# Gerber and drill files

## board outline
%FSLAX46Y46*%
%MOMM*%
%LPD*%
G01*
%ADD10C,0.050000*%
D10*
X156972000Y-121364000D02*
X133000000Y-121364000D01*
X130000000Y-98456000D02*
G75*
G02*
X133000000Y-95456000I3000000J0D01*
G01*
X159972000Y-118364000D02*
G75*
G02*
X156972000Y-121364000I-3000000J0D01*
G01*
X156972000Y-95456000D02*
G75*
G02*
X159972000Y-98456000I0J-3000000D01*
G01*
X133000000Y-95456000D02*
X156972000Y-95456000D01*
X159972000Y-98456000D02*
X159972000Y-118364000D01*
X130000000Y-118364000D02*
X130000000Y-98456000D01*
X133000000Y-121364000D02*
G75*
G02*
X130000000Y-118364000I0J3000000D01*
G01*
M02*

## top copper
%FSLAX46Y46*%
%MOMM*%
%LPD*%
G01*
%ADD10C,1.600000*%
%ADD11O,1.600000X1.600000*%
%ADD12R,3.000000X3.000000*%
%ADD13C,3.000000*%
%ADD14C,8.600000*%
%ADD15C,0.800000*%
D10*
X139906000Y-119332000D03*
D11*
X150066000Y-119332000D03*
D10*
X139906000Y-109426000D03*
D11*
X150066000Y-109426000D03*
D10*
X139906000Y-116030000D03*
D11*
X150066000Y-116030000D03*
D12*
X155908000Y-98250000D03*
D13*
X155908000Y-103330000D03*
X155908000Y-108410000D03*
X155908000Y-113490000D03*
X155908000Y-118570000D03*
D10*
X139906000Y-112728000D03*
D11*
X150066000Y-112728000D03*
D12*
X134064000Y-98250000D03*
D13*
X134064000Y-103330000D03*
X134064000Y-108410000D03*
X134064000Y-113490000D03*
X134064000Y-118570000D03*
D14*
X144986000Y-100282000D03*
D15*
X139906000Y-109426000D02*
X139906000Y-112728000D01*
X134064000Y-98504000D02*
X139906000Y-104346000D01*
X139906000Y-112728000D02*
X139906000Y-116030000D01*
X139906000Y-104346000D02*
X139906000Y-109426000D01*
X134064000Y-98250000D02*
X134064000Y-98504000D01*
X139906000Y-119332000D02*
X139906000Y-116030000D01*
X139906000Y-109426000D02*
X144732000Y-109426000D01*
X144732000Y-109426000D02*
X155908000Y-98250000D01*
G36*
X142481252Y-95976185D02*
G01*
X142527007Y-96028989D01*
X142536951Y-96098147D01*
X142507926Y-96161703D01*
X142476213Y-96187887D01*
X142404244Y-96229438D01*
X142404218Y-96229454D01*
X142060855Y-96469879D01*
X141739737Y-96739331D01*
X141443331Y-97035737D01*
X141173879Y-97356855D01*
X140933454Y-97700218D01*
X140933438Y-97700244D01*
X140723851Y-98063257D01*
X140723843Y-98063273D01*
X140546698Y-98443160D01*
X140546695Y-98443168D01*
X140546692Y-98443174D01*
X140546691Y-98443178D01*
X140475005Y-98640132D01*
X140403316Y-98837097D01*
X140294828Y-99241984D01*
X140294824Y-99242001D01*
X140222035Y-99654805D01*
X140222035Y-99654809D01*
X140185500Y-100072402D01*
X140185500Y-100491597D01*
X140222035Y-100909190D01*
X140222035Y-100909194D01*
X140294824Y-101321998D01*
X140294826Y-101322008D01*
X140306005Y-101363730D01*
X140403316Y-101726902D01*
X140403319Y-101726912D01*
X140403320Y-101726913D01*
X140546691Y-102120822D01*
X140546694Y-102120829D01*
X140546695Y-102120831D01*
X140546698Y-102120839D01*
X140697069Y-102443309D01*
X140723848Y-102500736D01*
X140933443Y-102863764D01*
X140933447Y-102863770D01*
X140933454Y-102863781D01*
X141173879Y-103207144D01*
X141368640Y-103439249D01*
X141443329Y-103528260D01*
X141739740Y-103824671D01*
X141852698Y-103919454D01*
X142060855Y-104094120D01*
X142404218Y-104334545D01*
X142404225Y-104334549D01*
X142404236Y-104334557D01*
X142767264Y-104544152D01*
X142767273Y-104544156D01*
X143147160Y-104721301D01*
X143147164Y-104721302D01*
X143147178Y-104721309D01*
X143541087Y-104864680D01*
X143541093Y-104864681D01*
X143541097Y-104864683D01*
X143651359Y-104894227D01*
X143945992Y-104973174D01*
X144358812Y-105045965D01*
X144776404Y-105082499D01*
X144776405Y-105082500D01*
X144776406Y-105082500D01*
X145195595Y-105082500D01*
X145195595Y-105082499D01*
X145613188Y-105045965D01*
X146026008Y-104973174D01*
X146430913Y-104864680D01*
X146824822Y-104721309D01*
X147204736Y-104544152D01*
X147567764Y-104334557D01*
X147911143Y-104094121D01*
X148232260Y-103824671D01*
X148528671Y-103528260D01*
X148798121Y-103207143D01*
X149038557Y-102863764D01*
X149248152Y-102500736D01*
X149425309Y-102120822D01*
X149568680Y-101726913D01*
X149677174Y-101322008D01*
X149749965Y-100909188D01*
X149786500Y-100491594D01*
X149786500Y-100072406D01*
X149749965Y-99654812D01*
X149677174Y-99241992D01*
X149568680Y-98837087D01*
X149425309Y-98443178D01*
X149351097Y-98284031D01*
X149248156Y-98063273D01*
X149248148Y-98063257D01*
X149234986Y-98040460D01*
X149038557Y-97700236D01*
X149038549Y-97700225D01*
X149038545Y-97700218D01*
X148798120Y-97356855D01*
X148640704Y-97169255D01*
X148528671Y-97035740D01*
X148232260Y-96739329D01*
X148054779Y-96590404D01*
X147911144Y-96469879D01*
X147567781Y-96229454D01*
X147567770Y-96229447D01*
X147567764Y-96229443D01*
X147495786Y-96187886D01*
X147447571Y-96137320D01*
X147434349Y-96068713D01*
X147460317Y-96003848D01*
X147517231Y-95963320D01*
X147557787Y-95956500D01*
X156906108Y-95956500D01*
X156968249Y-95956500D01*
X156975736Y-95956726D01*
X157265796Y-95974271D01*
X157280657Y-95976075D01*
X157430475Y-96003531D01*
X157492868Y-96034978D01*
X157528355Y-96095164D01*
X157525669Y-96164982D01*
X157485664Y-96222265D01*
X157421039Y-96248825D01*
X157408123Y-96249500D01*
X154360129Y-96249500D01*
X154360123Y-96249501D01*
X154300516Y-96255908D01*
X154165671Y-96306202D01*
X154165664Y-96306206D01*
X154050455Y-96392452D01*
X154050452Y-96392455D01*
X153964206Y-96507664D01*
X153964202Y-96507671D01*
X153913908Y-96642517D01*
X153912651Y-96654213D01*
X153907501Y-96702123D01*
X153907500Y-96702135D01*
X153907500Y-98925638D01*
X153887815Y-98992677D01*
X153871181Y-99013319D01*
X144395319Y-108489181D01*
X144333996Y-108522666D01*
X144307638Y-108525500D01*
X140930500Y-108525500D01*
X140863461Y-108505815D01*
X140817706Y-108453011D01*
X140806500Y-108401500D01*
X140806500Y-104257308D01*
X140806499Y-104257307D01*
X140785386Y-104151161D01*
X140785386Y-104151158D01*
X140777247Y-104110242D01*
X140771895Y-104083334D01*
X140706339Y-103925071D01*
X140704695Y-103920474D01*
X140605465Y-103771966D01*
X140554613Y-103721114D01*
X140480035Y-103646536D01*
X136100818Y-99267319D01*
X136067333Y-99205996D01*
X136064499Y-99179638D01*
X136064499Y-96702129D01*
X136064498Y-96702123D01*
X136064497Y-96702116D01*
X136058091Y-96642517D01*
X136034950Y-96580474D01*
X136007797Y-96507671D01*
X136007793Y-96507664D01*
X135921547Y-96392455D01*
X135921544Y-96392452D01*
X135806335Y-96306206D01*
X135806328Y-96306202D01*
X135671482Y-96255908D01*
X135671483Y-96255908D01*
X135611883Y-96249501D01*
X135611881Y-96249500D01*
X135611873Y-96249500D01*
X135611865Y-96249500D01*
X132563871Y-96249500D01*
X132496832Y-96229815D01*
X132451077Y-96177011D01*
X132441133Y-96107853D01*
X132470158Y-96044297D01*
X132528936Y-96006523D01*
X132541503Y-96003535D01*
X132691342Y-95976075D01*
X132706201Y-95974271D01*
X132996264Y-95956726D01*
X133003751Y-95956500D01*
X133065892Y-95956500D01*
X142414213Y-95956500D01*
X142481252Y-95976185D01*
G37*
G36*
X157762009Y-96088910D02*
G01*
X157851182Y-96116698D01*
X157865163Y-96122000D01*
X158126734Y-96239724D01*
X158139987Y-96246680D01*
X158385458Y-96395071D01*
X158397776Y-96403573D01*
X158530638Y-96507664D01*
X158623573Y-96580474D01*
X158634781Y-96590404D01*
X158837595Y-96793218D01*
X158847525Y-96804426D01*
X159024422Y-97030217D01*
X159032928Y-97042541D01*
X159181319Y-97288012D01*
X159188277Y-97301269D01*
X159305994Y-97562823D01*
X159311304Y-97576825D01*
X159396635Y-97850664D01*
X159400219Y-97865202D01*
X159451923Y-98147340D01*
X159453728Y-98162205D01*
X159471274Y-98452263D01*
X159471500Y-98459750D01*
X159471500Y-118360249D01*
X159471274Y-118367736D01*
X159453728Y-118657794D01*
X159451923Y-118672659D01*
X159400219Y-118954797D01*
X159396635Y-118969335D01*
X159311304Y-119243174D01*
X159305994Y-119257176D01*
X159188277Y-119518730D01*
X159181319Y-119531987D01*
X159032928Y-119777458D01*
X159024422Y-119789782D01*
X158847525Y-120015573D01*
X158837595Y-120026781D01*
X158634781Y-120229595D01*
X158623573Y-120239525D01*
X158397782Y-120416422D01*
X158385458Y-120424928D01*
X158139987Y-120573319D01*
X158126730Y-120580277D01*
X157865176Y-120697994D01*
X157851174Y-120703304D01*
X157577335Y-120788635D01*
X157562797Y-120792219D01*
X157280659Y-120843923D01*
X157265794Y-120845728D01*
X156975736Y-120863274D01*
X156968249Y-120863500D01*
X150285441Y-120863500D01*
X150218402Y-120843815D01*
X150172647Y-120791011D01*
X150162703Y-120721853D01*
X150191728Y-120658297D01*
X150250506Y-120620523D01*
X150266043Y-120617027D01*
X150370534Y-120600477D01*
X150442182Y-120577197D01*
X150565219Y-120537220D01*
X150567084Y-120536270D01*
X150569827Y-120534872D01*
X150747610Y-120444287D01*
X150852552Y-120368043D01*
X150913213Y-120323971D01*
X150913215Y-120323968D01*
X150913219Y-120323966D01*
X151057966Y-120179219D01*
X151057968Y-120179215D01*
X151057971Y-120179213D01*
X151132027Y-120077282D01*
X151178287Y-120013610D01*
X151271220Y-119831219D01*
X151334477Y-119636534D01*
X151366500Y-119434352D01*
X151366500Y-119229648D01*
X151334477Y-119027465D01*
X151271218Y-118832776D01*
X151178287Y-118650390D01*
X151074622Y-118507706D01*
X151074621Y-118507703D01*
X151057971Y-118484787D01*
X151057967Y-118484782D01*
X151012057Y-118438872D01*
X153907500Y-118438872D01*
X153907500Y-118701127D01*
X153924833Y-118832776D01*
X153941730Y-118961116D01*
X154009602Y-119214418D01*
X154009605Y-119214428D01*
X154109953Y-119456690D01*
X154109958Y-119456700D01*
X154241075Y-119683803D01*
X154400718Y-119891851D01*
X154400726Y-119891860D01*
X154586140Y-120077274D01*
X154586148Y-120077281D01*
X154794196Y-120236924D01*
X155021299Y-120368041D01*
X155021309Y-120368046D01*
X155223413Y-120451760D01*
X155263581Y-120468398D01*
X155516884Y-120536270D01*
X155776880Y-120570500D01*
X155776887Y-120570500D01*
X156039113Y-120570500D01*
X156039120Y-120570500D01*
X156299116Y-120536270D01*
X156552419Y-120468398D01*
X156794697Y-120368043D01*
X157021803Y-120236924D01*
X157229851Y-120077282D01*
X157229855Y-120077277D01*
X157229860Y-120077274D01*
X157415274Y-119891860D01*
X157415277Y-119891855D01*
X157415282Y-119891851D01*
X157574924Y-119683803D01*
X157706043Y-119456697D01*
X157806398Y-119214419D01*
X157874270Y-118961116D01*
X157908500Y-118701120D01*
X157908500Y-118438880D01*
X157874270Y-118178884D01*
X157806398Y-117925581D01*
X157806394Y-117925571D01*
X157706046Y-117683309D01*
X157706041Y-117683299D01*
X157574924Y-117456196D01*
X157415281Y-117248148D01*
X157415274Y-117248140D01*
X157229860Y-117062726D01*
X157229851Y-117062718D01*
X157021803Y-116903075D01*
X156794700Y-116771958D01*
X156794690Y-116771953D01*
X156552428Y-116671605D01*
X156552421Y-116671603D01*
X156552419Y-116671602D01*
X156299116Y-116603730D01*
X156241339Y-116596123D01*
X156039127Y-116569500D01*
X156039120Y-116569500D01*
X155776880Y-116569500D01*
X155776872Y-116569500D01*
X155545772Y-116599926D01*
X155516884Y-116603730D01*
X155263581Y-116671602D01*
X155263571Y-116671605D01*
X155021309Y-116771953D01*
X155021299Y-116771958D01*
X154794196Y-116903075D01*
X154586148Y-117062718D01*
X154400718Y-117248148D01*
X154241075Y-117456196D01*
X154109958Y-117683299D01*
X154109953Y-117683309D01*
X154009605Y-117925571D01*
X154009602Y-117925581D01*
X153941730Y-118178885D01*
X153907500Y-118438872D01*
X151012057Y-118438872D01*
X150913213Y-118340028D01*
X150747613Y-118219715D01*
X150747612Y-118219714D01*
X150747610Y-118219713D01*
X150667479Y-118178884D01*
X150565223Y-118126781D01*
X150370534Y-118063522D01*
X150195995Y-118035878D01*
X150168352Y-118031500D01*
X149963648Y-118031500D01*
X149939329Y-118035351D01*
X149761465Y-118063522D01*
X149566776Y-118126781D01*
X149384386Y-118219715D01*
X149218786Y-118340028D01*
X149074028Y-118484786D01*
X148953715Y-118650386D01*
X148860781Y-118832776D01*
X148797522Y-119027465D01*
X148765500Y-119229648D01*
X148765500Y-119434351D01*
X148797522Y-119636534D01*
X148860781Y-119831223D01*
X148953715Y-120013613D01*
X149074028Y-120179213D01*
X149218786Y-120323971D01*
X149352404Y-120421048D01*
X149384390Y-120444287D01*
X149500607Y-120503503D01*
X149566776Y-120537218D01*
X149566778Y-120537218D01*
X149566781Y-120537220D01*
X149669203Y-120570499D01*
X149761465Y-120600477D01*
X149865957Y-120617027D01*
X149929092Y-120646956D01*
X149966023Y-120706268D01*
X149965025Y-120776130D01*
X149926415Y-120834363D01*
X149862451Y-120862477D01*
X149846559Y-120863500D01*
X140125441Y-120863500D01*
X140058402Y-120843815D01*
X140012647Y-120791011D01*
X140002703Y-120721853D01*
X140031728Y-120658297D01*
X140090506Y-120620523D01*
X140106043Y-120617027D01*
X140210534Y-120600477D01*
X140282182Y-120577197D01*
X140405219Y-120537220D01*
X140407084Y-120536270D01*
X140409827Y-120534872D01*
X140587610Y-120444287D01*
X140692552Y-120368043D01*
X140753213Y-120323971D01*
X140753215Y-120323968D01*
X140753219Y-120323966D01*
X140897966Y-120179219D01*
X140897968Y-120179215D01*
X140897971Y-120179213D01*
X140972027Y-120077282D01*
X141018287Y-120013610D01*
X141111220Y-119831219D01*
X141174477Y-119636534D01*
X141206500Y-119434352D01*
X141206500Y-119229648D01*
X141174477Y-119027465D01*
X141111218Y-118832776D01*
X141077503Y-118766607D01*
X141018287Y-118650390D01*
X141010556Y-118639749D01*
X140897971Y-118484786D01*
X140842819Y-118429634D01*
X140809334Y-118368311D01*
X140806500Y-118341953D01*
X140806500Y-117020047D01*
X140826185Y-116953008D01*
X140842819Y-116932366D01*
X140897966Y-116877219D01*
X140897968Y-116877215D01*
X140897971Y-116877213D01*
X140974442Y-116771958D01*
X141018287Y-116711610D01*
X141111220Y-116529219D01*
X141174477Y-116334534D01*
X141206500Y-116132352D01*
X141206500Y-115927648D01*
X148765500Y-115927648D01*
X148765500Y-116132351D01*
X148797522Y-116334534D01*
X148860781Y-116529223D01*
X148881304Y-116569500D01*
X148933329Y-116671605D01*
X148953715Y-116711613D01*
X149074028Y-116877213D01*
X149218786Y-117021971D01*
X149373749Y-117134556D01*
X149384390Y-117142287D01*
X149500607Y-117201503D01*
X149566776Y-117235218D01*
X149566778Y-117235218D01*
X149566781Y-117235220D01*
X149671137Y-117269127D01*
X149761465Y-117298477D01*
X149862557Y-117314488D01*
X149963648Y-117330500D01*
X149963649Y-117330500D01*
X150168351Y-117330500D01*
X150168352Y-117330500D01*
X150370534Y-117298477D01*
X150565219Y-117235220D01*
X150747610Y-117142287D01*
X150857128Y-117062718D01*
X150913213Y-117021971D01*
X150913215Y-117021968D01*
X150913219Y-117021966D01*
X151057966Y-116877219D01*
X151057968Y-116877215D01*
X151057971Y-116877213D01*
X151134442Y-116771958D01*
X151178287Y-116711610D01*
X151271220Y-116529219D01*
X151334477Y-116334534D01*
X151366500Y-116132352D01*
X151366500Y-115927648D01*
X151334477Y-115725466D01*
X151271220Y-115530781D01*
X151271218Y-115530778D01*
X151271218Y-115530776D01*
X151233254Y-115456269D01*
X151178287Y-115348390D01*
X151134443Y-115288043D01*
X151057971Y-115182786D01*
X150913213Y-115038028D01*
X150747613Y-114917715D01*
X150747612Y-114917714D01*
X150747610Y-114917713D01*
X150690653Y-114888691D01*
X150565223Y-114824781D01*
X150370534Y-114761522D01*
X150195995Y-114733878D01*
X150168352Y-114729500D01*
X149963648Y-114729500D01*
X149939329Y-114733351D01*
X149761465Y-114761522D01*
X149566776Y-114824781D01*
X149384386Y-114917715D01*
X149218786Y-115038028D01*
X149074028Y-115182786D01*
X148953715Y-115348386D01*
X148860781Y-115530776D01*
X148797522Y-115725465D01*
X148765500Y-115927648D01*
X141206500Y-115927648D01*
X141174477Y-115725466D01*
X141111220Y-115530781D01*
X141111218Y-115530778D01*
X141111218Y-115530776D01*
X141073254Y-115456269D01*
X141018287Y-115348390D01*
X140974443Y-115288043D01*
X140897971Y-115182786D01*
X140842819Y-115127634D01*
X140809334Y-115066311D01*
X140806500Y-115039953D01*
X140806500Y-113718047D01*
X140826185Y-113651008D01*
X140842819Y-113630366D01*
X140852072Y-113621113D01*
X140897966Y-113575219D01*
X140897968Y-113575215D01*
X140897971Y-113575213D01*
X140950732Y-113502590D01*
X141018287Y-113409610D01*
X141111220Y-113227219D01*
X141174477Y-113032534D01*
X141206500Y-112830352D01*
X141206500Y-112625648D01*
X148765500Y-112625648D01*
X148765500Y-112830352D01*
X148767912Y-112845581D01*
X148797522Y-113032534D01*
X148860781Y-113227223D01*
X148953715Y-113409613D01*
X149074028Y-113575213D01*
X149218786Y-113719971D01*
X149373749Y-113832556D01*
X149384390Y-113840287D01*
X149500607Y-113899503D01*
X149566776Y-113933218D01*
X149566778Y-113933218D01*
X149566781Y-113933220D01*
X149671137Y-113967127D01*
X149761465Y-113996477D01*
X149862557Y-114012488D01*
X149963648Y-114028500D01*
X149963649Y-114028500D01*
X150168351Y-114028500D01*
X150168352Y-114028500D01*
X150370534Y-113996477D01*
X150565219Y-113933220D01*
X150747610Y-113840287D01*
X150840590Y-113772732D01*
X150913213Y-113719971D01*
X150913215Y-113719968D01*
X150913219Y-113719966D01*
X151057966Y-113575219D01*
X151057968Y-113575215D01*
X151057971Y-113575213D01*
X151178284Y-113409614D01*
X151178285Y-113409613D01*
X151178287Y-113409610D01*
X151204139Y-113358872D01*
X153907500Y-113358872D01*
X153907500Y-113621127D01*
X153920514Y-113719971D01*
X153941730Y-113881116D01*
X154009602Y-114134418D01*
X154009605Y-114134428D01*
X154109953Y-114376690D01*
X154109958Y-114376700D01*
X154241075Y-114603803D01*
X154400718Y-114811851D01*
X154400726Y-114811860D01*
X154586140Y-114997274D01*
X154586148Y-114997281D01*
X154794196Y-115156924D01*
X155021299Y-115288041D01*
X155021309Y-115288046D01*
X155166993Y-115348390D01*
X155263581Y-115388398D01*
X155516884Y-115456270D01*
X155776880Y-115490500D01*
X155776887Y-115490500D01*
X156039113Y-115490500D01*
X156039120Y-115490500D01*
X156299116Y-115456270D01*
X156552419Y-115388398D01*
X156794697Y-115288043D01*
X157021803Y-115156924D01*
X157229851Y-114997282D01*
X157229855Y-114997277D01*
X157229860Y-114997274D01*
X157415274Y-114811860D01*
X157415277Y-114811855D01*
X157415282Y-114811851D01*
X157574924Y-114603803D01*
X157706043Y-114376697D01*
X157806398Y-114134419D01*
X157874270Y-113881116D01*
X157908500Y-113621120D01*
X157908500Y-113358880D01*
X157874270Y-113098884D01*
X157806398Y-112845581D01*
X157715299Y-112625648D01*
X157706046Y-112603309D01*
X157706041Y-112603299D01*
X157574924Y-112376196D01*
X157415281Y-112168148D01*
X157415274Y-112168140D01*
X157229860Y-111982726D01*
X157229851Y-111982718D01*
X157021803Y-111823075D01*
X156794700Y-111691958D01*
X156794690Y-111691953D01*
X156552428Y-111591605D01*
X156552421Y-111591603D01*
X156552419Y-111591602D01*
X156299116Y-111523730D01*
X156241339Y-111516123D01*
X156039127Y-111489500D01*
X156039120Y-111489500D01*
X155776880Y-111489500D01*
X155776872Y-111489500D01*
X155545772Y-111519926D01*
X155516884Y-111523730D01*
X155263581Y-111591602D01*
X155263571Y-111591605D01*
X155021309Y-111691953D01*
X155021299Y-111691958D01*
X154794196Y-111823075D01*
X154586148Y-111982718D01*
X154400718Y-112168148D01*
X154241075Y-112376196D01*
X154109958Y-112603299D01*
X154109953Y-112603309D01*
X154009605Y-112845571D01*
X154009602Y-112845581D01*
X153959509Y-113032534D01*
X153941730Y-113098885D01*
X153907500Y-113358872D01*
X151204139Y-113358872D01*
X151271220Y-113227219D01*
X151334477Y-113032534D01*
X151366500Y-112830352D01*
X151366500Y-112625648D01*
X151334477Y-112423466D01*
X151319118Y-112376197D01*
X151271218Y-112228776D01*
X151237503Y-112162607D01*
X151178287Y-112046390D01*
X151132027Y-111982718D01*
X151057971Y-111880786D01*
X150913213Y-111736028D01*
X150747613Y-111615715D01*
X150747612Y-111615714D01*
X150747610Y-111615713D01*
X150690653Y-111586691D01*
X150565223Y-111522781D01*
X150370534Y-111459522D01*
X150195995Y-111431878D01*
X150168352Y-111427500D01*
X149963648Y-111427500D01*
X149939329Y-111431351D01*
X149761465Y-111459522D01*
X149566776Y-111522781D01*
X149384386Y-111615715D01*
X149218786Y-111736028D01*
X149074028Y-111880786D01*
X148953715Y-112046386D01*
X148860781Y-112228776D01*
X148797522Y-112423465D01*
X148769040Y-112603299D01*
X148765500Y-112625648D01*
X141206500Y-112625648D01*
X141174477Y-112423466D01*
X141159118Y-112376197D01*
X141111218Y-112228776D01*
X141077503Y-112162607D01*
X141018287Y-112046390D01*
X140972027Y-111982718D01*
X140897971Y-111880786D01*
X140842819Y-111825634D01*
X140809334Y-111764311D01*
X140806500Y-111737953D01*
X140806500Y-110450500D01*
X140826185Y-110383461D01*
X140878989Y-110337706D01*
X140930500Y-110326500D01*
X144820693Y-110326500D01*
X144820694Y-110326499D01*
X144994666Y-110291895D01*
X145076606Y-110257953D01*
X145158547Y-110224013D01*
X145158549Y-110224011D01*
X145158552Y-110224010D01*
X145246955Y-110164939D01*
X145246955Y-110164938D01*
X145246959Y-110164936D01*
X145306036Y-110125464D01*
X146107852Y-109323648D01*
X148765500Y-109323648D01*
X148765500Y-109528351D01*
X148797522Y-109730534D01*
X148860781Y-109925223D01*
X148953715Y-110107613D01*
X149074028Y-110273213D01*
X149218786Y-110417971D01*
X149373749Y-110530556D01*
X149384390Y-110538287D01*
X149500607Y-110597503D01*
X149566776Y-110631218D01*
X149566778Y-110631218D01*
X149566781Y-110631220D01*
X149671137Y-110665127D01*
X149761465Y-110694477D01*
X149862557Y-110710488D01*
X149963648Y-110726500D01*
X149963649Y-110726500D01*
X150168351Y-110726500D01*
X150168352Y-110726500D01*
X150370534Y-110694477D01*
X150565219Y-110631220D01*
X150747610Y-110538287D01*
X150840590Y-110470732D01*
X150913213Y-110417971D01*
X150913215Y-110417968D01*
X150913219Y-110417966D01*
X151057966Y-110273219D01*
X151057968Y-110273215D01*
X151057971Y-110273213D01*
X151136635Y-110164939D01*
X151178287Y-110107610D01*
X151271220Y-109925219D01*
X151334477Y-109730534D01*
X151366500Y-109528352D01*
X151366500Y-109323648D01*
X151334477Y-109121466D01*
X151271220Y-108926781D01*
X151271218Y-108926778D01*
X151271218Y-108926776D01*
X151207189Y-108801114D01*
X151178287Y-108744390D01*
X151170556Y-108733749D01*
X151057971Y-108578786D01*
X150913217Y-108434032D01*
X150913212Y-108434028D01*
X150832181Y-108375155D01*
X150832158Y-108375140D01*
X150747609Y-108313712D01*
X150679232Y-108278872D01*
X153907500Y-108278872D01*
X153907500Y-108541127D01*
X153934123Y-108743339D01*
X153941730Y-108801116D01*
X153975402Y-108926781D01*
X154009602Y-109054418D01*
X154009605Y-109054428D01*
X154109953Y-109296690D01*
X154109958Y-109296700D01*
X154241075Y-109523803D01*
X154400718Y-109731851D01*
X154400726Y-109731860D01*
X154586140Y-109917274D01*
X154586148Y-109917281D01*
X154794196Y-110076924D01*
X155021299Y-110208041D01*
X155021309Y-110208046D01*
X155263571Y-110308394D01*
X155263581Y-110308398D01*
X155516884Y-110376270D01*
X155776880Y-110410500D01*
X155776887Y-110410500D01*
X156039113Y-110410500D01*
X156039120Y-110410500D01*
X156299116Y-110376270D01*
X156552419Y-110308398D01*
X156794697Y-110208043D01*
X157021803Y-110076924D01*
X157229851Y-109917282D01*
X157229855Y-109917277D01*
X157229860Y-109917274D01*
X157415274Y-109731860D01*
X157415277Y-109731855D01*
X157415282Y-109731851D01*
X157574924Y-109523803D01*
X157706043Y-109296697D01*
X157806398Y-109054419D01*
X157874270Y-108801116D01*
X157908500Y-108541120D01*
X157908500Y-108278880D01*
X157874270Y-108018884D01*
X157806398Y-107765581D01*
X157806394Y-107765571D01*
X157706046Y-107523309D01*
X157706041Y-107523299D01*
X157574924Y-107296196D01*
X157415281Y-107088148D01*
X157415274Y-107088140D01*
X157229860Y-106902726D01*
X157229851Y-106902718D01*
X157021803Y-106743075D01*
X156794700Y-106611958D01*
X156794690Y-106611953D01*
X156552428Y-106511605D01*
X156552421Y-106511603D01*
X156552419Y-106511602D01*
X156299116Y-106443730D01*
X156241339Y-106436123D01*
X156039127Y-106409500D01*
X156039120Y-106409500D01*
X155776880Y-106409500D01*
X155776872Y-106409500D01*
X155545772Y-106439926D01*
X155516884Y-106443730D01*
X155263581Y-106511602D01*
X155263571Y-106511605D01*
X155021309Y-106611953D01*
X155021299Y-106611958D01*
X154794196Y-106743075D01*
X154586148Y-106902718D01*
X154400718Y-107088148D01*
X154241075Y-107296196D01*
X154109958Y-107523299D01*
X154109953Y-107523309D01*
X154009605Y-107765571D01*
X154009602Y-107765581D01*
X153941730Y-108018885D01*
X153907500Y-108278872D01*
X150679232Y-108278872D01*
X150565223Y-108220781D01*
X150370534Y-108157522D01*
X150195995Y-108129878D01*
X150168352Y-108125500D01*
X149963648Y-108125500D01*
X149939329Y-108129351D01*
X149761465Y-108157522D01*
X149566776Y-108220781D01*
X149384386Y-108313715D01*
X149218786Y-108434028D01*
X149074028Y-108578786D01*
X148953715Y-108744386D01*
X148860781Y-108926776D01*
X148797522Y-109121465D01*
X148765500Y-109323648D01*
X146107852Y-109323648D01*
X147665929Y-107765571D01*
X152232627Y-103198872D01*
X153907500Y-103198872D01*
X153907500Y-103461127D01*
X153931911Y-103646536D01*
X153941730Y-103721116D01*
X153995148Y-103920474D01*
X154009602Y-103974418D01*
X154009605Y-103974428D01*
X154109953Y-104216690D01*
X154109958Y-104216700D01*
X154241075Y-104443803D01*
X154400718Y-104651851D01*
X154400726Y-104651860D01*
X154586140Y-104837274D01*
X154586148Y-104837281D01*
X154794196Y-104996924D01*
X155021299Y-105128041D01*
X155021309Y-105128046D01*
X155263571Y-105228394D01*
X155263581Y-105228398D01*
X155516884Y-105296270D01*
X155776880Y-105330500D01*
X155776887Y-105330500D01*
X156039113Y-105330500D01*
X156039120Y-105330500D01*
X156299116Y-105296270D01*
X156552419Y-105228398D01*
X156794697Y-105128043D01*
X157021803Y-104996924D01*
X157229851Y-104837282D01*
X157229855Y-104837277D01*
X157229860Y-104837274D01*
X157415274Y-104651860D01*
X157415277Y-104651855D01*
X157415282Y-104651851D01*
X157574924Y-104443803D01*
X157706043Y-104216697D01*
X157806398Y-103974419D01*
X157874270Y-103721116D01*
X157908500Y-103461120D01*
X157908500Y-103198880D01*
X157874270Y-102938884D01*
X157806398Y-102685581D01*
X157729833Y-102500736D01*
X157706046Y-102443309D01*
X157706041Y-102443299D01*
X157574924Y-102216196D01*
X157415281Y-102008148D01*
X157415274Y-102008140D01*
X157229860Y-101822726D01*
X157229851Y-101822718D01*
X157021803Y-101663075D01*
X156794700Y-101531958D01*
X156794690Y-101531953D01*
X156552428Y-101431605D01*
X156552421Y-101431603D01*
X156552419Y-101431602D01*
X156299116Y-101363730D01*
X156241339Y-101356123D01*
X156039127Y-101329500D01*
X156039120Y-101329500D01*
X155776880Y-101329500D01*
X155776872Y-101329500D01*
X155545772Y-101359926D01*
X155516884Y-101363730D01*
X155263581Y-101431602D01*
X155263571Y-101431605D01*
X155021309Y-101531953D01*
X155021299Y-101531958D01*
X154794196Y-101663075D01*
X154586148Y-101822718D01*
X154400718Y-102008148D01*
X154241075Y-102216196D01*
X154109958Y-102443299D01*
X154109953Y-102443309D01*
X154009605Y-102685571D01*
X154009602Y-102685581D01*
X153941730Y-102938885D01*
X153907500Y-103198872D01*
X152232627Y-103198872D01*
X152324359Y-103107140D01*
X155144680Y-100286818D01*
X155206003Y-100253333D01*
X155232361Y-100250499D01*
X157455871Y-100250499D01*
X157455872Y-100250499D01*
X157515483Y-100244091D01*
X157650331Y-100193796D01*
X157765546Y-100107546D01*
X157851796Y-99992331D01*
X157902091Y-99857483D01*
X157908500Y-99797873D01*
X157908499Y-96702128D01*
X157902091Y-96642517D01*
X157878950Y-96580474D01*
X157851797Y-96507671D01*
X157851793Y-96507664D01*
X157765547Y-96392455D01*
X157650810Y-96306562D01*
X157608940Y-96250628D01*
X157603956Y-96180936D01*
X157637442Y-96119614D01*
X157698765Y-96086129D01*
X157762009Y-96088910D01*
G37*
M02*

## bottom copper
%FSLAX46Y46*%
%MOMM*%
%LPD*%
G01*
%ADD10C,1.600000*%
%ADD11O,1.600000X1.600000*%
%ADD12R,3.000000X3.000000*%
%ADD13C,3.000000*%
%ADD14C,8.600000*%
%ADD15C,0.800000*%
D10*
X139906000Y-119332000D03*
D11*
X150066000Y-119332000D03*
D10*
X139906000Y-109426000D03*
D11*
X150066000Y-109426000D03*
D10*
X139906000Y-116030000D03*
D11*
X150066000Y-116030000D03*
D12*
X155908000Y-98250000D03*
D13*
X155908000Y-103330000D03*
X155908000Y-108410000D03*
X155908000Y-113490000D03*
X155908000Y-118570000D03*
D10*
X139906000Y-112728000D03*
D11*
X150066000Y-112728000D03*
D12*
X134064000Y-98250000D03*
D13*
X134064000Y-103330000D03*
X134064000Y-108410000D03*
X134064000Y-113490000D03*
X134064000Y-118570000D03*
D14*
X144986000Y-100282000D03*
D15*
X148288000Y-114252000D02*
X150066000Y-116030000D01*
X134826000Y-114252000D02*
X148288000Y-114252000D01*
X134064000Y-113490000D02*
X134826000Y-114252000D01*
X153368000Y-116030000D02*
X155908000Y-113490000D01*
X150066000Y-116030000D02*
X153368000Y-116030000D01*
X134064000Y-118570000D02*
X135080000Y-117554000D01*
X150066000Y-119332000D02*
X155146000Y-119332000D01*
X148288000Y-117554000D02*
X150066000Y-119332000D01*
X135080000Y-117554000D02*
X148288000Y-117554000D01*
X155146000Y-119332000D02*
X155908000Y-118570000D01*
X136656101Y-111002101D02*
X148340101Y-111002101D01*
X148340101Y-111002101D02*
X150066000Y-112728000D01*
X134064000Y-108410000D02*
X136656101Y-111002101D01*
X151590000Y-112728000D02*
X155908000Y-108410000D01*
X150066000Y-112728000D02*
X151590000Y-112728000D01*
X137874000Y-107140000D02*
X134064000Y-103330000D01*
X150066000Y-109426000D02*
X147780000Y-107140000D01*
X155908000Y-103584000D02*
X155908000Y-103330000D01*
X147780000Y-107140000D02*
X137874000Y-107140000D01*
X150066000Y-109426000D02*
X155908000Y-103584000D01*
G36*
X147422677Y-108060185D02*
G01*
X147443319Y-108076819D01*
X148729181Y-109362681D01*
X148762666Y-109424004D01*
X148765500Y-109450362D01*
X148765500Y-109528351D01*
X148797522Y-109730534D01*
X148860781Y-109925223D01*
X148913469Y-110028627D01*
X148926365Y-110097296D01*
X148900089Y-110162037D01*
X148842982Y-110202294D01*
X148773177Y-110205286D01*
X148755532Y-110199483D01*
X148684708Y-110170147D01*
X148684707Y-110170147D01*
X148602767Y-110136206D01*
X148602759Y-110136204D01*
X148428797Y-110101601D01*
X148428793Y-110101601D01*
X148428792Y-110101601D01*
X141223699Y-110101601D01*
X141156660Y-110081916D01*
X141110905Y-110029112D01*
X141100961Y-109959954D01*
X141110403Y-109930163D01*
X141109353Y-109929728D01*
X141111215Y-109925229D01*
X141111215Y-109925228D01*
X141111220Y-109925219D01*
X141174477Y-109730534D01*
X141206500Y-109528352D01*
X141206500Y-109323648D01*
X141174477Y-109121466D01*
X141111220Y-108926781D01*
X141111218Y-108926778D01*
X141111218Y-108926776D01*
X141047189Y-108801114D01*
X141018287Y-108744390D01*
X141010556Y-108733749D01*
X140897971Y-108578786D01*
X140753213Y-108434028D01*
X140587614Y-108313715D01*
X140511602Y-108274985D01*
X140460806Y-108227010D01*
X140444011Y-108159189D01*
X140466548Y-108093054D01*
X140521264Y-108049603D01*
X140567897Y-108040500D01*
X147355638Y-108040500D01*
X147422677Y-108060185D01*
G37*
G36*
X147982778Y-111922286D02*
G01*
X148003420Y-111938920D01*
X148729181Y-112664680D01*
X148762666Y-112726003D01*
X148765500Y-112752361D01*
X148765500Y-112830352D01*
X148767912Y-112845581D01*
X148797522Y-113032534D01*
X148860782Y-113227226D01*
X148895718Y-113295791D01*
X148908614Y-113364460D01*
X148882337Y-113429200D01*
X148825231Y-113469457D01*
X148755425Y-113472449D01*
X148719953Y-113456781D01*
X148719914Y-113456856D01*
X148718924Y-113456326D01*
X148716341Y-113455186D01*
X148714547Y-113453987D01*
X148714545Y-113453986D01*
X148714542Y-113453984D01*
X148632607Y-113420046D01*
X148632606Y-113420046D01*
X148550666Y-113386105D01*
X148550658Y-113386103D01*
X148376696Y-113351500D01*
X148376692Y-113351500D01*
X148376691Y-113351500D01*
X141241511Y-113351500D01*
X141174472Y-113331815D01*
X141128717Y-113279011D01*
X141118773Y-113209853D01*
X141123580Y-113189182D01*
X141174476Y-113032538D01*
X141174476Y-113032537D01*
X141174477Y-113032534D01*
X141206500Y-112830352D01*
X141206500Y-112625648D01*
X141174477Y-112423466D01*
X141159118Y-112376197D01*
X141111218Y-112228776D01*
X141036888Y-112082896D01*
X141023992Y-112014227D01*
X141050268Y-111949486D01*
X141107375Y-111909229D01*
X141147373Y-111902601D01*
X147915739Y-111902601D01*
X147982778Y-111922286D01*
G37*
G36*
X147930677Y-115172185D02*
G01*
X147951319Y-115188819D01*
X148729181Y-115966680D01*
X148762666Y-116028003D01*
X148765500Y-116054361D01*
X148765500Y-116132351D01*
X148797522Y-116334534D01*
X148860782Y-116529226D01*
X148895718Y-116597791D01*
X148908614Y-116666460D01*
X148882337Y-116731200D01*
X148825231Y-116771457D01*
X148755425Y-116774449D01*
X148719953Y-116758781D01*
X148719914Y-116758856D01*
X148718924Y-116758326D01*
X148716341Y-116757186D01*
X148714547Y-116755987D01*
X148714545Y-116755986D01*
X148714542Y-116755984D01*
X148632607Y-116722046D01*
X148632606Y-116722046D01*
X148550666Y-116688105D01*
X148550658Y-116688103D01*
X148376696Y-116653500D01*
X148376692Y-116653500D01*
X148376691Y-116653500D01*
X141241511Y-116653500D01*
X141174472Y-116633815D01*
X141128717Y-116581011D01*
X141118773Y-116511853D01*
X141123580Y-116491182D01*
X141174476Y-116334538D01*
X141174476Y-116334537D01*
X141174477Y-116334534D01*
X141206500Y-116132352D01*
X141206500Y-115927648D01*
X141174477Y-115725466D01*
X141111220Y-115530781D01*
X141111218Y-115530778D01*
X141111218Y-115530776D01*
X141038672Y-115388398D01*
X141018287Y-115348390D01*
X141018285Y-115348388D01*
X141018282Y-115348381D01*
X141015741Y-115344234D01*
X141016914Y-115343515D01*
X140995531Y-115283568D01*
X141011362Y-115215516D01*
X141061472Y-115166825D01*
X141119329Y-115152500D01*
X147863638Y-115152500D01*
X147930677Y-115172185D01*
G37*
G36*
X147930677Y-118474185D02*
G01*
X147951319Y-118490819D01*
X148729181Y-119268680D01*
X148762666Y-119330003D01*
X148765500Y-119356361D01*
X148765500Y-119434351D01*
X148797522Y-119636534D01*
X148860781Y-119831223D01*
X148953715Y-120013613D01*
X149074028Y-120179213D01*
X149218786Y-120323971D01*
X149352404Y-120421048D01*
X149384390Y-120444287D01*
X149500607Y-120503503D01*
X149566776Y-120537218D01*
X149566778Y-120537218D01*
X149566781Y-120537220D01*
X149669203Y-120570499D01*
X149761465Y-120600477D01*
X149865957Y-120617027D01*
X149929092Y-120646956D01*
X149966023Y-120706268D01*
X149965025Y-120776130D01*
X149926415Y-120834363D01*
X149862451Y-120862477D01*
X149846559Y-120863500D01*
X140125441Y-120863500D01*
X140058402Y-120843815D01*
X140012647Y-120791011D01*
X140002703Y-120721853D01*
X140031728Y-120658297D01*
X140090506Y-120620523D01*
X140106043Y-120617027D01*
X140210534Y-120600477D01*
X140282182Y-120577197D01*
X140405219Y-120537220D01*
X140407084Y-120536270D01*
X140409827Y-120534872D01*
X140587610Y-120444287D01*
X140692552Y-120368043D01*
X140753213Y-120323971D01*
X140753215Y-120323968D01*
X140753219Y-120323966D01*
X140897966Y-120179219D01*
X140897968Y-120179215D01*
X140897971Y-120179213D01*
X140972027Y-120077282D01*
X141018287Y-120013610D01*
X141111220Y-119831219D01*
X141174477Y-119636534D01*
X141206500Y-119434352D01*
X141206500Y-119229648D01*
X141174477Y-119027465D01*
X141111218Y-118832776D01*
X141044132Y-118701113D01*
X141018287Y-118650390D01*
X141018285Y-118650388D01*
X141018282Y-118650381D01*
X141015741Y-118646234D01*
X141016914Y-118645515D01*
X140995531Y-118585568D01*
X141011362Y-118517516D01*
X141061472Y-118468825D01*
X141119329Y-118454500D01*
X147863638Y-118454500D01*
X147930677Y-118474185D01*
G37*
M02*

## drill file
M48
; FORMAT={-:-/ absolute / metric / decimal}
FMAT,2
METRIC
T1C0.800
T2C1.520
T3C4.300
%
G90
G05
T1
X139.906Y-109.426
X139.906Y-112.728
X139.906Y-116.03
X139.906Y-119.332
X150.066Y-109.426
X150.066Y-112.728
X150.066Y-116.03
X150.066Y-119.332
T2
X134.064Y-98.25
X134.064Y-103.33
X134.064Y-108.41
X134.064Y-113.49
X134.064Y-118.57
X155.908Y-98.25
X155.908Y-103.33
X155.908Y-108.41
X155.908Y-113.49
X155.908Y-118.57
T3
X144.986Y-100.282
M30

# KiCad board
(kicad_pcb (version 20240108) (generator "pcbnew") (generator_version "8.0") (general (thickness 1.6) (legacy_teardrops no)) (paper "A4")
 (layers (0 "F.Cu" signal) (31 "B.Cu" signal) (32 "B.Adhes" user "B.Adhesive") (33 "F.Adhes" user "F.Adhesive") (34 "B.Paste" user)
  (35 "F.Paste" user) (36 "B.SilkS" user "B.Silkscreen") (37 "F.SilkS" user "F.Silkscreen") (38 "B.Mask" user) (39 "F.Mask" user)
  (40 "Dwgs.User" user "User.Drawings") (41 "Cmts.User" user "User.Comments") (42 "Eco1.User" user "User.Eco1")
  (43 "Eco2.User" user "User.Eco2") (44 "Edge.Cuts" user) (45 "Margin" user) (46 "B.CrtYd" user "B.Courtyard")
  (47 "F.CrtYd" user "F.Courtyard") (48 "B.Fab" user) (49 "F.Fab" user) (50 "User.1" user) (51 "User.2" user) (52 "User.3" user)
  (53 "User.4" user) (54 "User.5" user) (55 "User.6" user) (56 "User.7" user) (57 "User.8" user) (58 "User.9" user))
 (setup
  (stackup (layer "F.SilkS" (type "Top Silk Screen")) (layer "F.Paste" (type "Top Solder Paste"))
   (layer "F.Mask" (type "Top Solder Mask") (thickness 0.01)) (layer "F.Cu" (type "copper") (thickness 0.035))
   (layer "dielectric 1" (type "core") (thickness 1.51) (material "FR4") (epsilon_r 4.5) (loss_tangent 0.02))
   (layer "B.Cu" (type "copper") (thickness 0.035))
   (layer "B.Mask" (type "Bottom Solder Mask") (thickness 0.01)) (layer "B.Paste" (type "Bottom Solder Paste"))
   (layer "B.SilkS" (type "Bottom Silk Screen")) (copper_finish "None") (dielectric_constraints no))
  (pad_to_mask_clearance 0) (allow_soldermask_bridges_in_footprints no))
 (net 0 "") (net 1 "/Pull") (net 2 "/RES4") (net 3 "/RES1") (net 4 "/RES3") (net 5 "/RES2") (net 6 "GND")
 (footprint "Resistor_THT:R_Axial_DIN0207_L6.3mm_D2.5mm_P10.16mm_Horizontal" (layer "F.Cu") (at 139.906 119.332)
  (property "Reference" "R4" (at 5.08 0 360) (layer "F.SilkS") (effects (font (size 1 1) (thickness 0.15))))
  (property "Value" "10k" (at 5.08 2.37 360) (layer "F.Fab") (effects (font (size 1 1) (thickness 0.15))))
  (pad "1" thru_hole circle (at 0 0) (size 1.6 1.6) (drill 0.8) (layers "*.Cu" "*.Mask") (remove_unused_layers no) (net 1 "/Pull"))
  (pad "2" thru_hole oval (at 10.16 0) (size 1.6 1.6) (drill 0.8) (layers "*.Cu" "*.Mask") (remove_unused_layers no) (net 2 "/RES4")))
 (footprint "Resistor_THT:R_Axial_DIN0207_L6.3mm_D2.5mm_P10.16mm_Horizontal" (layer "F.Cu") (at 139.906 109.426)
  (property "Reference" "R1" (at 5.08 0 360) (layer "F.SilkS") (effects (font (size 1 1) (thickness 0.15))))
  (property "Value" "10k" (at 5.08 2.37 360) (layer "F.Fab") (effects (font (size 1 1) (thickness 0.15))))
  (pad "1" thru_hole circle (at 0 0) (size 1.6 1.6) (drill 0.8) (layers "*.Cu" "*.Mask") (remove_unused_layers no) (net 1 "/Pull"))
  (pad "2" thru_hole oval (at 10.16 0) (size 1.6 1.6) (drill 0.8) (layers "*.Cu" "*.Mask") (remove_unused_layers no) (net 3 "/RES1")))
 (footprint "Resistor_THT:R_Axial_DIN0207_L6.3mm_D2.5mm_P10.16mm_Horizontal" (layer "F.Cu") (at 139.906 116.03)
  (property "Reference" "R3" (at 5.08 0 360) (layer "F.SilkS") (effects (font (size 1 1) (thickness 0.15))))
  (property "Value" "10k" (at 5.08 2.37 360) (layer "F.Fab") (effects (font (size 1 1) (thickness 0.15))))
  (pad "1" thru_hole circle (at 0 0) (size 1.6 1.6) (drill 0.8) (layers "*.Cu" "*.Mask") (remove_unused_layers no) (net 1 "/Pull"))
  (pad "2" thru_hole oval (at 10.16 0) (size 1.6 1.6) (drill 0.8) (layers "*.Cu" "*.Mask") (remove_unused_layers no) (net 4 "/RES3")))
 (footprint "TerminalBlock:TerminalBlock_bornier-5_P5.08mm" (layer "F.Cu") (at 155.908 98.25 -90)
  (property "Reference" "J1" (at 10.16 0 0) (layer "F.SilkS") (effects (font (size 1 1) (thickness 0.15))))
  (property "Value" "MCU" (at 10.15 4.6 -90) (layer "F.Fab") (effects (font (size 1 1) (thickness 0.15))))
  (pad "1" thru_hole rect (at 0 0 270) (size 3 3) (drill 1.52) (layers "*.Cu" "*.Mask") (remove_unused_layers no) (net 1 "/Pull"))
  (pad "2" thru_hole circle (at 5.08 0 270) (size 3 3) (drill 1.52) (layers "*.Cu" "*.Mask") (remove_unused_layers no) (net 3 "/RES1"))
  (pad "3" thru_hole circle (at 10.16 0 270) (size 3 3) (drill 1.52) (layers "*.Cu" "*.Mask") (remove_unused_layers no) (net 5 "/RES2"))
  (pad "4" thru_hole circle (at 15.24 0 270) (size 3 3) (drill 1.52) (layers "*.Cu" "*.Mask") (remove_unused_layers no) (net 4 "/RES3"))
  (pad "5" thru_hole circle (at 20.32 0 270) (size 3 3) (drill 1.52) (layers "*.Cu" "*.Mask") (remove_unused_layers no) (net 2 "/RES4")))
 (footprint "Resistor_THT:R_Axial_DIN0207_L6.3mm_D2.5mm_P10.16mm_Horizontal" (layer "F.Cu") (at 139.906 112.728)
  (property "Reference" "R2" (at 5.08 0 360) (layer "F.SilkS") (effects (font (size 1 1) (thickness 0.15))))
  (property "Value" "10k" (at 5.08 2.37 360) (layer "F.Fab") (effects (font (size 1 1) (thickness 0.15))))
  (pad "1" thru_hole circle (at 0 0) (size 1.6 1.6) (drill 0.8) (layers "*.Cu" "*.Mask") (remove_unused_layers no) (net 1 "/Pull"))
  (pad "2" thru_hole oval (at 10.16 0) (size 1.6 1.6) (drill 0.8) (layers "*.Cu" "*.Mask") (remove_unused_layers no) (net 5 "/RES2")))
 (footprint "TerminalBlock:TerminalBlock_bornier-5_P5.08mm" (layer "F.Cu") (at 134.064 98.25 -90)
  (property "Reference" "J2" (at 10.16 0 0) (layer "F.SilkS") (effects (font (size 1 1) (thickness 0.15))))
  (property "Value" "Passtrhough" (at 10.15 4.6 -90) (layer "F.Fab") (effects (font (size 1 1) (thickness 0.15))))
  (pad "1" thru_hole rect (at 0 0 270) (size 3 3) (drill 1.52) (layers "*.Cu" "*.Mask") (remove_unused_layers no) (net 1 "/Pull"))
  (pad "2" thru_hole circle (at 5.08 0 270) (size 3 3) (drill 1.52) (layers "*.Cu" "*.Mask") (remove_unused_layers no) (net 3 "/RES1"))
  (pad "3" thru_hole circle (at 10.16 0 270) (size 3 3) (drill 1.52) (layers "*.Cu" "*.Mask") (remove_unused_layers no) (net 5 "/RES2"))
  (pad "4" thru_hole circle (at 15.24 0 270) (size 3 3) (drill 1.52) (layers "*.Cu" "*.Mask") (remove_unused_layers no) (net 4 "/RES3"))
  (pad "5" thru_hole circle (at 20.32 0 270) (size 3 3) (drill 1.52) (layers "*.Cu" "*.Mask") (remove_unused_layers no) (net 2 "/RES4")))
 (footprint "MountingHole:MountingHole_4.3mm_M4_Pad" (layer "F.Cu") (at 144.986 100.282)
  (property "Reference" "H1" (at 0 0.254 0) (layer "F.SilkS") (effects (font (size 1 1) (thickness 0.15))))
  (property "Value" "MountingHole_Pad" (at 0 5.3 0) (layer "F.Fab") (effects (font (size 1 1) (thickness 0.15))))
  (pad "1" thru_hole circle (at 0 0) (size 8.6 8.6) (drill 4.3) (layers "*.Cu" "*.Mask") (remove_unused_layers no) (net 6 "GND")))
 (gr_line (start 156.972 121.364) (end 133 121.364) (stroke (width 0.05) (type default)) (layer "Edge.Cuts"))
 (gr_arc (start 130 98.456) (mid 130.87868 96.33468) (end 133 95.456) (stroke (width 0.05) (type default)) (layer "Edge.Cuts"))
 (gr_arc (start 159.972 118.364) (mid 159.09332 120.48532) (end 156.972 121.364) (stroke (width 0.05) (type default)) (layer "Edge.Cuts"))
 (gr_arc (start 156.972 95.456) (mid 159.09332 96.33468) (end 159.972 98.456) (stroke (width 0.05) (type default)) (layer "Edge.Cuts"))
 (gr_line (start 133 95.456) (end 156.972 95.456) (stroke (width 0.05) (type default)) (layer "Edge.Cuts"))
 (gr_line (start 159.972 98.456) (end 159.972 118.364) (stroke (width 0.05) (type default)) (layer "Edge.Cuts"))
 (gr_line (start 130 118.364) (end 130 98.456) (stroke (width 0.05) (type default)) (layer "Edge.Cuts"))
 (gr_arc (start 133 121.364) (mid 130.87868 120.48532) (end 130 118.364) (stroke (width 0.05) (type default)) (layer "Edge.Cuts"))
 (segment (start 148.288 114.252) (end 150.066 116.03) (width 0.8) (layer "B.Cu") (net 4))
 (segment (start 134.826 114.252) (end 148.288 114.252) (width 0.8) (layer "B.Cu") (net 4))
 (segment (start 134.064 113.49) (end 134.826 114.252) (width 0.8) (layer "B.Cu") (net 4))
 (segment (start 153.368 116.03) (end 155.908 113.49) (width 0.8) (layer "B.Cu") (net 4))
 (segment (start 150.066 116.03) (end 153.368 116.03) (width 0.8) (layer "B.Cu") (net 4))
 (segment (start 134.064 118.57) (end 135.08 117.554) (width 0.8) (layer "B.Cu") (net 2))
 (segment (start 150.066 119.332) (end 155.146 119.332) (width 0.8) (layer "B.Cu") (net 2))
 (segment (start 148.288 117.554) (end 150.066 119.332) (width 0.8) (layer "B.Cu") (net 2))
 (segment (start 135.08 117.554) (end 148.288 117.554) (width 0.8) (layer "B.Cu") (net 2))
 (segment (start 155.146 119.332) (end 155.908 118.57) (width 0.8) (layer "B.Cu") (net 2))
 (segment (start 136.656101 111.002101) (end 148.340101 111.002101) (width 0.8) (layer "B.Cu") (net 5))
 (segment (start 148.340101 111.002101) (end 150.066 112.728) (width 0.8) (layer "B.Cu") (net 5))
 (segment (start 134.064 108.41) (end 136.656101 111.002101) (width 0.8) (layer "B.Cu") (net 5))
 (segment (start 151.59 112.728) (end 155.908 108.41) (width 0.8) (layer "B.Cu") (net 5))
 (segment (start 150.066 112.728) (end 151.59 112.728) (width 0.8) (layer "B.Cu") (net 5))
 (segment (start 137.874 107.14) (end 134.064 103.33) (width 0.8) (layer "B.Cu") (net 3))
 (segment (start 150.066 109.426) (end 147.78 107.14) (width 0.8) (layer "B.Cu") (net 3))
 (segment (start 155.908 103.584) (end 155.908 103.33) (width 0.8) (layer "B.Cu") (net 3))
 (segment (start 147.78 107.14) (end 137.874 107.14) (width 0.8) (layer "B.Cu") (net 3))
 (segment (start 150.066 109.426) (end 155.908 103.584) (width 0.8) (layer "B.Cu") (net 3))
 (segment (start 139.906 109.426) (end 139.906 112.728) (width 0.8) (layer "F.Cu") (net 1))
 (segment (start 134.064 98.504) (end 139.906 104.346) (width 0.8) (layer "F.Cu") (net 1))
 (segment (start 139.906 112.728) (end 139.906 116.03) (width 0.8) (layer "F.Cu") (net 1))
 (segment (start 139.906 104.346) (end 139.906 109.426) (width 0.8) (layer "F.Cu") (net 1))
 (segment (start 134.064 98.25) (end 134.064 98.504) (width 0.8) (layer "F.Cu") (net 1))
 (segment (start 139.906 119.332) (end 139.906 116.03) (width 0.8) (layer "F.Cu") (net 1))
 (segment (start 139.906 109.426) (end 144.732 109.426) (width 0.8) (layer "F.Cu") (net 1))
 (segment (start 144.732 109.426) (end 155.908 98.25) (width 0.8) (layer "F.Cu") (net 1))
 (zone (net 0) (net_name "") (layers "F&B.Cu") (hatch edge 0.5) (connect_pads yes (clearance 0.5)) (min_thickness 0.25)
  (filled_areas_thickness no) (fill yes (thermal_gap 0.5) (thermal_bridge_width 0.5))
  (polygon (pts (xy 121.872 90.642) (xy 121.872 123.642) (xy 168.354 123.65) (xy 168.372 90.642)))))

